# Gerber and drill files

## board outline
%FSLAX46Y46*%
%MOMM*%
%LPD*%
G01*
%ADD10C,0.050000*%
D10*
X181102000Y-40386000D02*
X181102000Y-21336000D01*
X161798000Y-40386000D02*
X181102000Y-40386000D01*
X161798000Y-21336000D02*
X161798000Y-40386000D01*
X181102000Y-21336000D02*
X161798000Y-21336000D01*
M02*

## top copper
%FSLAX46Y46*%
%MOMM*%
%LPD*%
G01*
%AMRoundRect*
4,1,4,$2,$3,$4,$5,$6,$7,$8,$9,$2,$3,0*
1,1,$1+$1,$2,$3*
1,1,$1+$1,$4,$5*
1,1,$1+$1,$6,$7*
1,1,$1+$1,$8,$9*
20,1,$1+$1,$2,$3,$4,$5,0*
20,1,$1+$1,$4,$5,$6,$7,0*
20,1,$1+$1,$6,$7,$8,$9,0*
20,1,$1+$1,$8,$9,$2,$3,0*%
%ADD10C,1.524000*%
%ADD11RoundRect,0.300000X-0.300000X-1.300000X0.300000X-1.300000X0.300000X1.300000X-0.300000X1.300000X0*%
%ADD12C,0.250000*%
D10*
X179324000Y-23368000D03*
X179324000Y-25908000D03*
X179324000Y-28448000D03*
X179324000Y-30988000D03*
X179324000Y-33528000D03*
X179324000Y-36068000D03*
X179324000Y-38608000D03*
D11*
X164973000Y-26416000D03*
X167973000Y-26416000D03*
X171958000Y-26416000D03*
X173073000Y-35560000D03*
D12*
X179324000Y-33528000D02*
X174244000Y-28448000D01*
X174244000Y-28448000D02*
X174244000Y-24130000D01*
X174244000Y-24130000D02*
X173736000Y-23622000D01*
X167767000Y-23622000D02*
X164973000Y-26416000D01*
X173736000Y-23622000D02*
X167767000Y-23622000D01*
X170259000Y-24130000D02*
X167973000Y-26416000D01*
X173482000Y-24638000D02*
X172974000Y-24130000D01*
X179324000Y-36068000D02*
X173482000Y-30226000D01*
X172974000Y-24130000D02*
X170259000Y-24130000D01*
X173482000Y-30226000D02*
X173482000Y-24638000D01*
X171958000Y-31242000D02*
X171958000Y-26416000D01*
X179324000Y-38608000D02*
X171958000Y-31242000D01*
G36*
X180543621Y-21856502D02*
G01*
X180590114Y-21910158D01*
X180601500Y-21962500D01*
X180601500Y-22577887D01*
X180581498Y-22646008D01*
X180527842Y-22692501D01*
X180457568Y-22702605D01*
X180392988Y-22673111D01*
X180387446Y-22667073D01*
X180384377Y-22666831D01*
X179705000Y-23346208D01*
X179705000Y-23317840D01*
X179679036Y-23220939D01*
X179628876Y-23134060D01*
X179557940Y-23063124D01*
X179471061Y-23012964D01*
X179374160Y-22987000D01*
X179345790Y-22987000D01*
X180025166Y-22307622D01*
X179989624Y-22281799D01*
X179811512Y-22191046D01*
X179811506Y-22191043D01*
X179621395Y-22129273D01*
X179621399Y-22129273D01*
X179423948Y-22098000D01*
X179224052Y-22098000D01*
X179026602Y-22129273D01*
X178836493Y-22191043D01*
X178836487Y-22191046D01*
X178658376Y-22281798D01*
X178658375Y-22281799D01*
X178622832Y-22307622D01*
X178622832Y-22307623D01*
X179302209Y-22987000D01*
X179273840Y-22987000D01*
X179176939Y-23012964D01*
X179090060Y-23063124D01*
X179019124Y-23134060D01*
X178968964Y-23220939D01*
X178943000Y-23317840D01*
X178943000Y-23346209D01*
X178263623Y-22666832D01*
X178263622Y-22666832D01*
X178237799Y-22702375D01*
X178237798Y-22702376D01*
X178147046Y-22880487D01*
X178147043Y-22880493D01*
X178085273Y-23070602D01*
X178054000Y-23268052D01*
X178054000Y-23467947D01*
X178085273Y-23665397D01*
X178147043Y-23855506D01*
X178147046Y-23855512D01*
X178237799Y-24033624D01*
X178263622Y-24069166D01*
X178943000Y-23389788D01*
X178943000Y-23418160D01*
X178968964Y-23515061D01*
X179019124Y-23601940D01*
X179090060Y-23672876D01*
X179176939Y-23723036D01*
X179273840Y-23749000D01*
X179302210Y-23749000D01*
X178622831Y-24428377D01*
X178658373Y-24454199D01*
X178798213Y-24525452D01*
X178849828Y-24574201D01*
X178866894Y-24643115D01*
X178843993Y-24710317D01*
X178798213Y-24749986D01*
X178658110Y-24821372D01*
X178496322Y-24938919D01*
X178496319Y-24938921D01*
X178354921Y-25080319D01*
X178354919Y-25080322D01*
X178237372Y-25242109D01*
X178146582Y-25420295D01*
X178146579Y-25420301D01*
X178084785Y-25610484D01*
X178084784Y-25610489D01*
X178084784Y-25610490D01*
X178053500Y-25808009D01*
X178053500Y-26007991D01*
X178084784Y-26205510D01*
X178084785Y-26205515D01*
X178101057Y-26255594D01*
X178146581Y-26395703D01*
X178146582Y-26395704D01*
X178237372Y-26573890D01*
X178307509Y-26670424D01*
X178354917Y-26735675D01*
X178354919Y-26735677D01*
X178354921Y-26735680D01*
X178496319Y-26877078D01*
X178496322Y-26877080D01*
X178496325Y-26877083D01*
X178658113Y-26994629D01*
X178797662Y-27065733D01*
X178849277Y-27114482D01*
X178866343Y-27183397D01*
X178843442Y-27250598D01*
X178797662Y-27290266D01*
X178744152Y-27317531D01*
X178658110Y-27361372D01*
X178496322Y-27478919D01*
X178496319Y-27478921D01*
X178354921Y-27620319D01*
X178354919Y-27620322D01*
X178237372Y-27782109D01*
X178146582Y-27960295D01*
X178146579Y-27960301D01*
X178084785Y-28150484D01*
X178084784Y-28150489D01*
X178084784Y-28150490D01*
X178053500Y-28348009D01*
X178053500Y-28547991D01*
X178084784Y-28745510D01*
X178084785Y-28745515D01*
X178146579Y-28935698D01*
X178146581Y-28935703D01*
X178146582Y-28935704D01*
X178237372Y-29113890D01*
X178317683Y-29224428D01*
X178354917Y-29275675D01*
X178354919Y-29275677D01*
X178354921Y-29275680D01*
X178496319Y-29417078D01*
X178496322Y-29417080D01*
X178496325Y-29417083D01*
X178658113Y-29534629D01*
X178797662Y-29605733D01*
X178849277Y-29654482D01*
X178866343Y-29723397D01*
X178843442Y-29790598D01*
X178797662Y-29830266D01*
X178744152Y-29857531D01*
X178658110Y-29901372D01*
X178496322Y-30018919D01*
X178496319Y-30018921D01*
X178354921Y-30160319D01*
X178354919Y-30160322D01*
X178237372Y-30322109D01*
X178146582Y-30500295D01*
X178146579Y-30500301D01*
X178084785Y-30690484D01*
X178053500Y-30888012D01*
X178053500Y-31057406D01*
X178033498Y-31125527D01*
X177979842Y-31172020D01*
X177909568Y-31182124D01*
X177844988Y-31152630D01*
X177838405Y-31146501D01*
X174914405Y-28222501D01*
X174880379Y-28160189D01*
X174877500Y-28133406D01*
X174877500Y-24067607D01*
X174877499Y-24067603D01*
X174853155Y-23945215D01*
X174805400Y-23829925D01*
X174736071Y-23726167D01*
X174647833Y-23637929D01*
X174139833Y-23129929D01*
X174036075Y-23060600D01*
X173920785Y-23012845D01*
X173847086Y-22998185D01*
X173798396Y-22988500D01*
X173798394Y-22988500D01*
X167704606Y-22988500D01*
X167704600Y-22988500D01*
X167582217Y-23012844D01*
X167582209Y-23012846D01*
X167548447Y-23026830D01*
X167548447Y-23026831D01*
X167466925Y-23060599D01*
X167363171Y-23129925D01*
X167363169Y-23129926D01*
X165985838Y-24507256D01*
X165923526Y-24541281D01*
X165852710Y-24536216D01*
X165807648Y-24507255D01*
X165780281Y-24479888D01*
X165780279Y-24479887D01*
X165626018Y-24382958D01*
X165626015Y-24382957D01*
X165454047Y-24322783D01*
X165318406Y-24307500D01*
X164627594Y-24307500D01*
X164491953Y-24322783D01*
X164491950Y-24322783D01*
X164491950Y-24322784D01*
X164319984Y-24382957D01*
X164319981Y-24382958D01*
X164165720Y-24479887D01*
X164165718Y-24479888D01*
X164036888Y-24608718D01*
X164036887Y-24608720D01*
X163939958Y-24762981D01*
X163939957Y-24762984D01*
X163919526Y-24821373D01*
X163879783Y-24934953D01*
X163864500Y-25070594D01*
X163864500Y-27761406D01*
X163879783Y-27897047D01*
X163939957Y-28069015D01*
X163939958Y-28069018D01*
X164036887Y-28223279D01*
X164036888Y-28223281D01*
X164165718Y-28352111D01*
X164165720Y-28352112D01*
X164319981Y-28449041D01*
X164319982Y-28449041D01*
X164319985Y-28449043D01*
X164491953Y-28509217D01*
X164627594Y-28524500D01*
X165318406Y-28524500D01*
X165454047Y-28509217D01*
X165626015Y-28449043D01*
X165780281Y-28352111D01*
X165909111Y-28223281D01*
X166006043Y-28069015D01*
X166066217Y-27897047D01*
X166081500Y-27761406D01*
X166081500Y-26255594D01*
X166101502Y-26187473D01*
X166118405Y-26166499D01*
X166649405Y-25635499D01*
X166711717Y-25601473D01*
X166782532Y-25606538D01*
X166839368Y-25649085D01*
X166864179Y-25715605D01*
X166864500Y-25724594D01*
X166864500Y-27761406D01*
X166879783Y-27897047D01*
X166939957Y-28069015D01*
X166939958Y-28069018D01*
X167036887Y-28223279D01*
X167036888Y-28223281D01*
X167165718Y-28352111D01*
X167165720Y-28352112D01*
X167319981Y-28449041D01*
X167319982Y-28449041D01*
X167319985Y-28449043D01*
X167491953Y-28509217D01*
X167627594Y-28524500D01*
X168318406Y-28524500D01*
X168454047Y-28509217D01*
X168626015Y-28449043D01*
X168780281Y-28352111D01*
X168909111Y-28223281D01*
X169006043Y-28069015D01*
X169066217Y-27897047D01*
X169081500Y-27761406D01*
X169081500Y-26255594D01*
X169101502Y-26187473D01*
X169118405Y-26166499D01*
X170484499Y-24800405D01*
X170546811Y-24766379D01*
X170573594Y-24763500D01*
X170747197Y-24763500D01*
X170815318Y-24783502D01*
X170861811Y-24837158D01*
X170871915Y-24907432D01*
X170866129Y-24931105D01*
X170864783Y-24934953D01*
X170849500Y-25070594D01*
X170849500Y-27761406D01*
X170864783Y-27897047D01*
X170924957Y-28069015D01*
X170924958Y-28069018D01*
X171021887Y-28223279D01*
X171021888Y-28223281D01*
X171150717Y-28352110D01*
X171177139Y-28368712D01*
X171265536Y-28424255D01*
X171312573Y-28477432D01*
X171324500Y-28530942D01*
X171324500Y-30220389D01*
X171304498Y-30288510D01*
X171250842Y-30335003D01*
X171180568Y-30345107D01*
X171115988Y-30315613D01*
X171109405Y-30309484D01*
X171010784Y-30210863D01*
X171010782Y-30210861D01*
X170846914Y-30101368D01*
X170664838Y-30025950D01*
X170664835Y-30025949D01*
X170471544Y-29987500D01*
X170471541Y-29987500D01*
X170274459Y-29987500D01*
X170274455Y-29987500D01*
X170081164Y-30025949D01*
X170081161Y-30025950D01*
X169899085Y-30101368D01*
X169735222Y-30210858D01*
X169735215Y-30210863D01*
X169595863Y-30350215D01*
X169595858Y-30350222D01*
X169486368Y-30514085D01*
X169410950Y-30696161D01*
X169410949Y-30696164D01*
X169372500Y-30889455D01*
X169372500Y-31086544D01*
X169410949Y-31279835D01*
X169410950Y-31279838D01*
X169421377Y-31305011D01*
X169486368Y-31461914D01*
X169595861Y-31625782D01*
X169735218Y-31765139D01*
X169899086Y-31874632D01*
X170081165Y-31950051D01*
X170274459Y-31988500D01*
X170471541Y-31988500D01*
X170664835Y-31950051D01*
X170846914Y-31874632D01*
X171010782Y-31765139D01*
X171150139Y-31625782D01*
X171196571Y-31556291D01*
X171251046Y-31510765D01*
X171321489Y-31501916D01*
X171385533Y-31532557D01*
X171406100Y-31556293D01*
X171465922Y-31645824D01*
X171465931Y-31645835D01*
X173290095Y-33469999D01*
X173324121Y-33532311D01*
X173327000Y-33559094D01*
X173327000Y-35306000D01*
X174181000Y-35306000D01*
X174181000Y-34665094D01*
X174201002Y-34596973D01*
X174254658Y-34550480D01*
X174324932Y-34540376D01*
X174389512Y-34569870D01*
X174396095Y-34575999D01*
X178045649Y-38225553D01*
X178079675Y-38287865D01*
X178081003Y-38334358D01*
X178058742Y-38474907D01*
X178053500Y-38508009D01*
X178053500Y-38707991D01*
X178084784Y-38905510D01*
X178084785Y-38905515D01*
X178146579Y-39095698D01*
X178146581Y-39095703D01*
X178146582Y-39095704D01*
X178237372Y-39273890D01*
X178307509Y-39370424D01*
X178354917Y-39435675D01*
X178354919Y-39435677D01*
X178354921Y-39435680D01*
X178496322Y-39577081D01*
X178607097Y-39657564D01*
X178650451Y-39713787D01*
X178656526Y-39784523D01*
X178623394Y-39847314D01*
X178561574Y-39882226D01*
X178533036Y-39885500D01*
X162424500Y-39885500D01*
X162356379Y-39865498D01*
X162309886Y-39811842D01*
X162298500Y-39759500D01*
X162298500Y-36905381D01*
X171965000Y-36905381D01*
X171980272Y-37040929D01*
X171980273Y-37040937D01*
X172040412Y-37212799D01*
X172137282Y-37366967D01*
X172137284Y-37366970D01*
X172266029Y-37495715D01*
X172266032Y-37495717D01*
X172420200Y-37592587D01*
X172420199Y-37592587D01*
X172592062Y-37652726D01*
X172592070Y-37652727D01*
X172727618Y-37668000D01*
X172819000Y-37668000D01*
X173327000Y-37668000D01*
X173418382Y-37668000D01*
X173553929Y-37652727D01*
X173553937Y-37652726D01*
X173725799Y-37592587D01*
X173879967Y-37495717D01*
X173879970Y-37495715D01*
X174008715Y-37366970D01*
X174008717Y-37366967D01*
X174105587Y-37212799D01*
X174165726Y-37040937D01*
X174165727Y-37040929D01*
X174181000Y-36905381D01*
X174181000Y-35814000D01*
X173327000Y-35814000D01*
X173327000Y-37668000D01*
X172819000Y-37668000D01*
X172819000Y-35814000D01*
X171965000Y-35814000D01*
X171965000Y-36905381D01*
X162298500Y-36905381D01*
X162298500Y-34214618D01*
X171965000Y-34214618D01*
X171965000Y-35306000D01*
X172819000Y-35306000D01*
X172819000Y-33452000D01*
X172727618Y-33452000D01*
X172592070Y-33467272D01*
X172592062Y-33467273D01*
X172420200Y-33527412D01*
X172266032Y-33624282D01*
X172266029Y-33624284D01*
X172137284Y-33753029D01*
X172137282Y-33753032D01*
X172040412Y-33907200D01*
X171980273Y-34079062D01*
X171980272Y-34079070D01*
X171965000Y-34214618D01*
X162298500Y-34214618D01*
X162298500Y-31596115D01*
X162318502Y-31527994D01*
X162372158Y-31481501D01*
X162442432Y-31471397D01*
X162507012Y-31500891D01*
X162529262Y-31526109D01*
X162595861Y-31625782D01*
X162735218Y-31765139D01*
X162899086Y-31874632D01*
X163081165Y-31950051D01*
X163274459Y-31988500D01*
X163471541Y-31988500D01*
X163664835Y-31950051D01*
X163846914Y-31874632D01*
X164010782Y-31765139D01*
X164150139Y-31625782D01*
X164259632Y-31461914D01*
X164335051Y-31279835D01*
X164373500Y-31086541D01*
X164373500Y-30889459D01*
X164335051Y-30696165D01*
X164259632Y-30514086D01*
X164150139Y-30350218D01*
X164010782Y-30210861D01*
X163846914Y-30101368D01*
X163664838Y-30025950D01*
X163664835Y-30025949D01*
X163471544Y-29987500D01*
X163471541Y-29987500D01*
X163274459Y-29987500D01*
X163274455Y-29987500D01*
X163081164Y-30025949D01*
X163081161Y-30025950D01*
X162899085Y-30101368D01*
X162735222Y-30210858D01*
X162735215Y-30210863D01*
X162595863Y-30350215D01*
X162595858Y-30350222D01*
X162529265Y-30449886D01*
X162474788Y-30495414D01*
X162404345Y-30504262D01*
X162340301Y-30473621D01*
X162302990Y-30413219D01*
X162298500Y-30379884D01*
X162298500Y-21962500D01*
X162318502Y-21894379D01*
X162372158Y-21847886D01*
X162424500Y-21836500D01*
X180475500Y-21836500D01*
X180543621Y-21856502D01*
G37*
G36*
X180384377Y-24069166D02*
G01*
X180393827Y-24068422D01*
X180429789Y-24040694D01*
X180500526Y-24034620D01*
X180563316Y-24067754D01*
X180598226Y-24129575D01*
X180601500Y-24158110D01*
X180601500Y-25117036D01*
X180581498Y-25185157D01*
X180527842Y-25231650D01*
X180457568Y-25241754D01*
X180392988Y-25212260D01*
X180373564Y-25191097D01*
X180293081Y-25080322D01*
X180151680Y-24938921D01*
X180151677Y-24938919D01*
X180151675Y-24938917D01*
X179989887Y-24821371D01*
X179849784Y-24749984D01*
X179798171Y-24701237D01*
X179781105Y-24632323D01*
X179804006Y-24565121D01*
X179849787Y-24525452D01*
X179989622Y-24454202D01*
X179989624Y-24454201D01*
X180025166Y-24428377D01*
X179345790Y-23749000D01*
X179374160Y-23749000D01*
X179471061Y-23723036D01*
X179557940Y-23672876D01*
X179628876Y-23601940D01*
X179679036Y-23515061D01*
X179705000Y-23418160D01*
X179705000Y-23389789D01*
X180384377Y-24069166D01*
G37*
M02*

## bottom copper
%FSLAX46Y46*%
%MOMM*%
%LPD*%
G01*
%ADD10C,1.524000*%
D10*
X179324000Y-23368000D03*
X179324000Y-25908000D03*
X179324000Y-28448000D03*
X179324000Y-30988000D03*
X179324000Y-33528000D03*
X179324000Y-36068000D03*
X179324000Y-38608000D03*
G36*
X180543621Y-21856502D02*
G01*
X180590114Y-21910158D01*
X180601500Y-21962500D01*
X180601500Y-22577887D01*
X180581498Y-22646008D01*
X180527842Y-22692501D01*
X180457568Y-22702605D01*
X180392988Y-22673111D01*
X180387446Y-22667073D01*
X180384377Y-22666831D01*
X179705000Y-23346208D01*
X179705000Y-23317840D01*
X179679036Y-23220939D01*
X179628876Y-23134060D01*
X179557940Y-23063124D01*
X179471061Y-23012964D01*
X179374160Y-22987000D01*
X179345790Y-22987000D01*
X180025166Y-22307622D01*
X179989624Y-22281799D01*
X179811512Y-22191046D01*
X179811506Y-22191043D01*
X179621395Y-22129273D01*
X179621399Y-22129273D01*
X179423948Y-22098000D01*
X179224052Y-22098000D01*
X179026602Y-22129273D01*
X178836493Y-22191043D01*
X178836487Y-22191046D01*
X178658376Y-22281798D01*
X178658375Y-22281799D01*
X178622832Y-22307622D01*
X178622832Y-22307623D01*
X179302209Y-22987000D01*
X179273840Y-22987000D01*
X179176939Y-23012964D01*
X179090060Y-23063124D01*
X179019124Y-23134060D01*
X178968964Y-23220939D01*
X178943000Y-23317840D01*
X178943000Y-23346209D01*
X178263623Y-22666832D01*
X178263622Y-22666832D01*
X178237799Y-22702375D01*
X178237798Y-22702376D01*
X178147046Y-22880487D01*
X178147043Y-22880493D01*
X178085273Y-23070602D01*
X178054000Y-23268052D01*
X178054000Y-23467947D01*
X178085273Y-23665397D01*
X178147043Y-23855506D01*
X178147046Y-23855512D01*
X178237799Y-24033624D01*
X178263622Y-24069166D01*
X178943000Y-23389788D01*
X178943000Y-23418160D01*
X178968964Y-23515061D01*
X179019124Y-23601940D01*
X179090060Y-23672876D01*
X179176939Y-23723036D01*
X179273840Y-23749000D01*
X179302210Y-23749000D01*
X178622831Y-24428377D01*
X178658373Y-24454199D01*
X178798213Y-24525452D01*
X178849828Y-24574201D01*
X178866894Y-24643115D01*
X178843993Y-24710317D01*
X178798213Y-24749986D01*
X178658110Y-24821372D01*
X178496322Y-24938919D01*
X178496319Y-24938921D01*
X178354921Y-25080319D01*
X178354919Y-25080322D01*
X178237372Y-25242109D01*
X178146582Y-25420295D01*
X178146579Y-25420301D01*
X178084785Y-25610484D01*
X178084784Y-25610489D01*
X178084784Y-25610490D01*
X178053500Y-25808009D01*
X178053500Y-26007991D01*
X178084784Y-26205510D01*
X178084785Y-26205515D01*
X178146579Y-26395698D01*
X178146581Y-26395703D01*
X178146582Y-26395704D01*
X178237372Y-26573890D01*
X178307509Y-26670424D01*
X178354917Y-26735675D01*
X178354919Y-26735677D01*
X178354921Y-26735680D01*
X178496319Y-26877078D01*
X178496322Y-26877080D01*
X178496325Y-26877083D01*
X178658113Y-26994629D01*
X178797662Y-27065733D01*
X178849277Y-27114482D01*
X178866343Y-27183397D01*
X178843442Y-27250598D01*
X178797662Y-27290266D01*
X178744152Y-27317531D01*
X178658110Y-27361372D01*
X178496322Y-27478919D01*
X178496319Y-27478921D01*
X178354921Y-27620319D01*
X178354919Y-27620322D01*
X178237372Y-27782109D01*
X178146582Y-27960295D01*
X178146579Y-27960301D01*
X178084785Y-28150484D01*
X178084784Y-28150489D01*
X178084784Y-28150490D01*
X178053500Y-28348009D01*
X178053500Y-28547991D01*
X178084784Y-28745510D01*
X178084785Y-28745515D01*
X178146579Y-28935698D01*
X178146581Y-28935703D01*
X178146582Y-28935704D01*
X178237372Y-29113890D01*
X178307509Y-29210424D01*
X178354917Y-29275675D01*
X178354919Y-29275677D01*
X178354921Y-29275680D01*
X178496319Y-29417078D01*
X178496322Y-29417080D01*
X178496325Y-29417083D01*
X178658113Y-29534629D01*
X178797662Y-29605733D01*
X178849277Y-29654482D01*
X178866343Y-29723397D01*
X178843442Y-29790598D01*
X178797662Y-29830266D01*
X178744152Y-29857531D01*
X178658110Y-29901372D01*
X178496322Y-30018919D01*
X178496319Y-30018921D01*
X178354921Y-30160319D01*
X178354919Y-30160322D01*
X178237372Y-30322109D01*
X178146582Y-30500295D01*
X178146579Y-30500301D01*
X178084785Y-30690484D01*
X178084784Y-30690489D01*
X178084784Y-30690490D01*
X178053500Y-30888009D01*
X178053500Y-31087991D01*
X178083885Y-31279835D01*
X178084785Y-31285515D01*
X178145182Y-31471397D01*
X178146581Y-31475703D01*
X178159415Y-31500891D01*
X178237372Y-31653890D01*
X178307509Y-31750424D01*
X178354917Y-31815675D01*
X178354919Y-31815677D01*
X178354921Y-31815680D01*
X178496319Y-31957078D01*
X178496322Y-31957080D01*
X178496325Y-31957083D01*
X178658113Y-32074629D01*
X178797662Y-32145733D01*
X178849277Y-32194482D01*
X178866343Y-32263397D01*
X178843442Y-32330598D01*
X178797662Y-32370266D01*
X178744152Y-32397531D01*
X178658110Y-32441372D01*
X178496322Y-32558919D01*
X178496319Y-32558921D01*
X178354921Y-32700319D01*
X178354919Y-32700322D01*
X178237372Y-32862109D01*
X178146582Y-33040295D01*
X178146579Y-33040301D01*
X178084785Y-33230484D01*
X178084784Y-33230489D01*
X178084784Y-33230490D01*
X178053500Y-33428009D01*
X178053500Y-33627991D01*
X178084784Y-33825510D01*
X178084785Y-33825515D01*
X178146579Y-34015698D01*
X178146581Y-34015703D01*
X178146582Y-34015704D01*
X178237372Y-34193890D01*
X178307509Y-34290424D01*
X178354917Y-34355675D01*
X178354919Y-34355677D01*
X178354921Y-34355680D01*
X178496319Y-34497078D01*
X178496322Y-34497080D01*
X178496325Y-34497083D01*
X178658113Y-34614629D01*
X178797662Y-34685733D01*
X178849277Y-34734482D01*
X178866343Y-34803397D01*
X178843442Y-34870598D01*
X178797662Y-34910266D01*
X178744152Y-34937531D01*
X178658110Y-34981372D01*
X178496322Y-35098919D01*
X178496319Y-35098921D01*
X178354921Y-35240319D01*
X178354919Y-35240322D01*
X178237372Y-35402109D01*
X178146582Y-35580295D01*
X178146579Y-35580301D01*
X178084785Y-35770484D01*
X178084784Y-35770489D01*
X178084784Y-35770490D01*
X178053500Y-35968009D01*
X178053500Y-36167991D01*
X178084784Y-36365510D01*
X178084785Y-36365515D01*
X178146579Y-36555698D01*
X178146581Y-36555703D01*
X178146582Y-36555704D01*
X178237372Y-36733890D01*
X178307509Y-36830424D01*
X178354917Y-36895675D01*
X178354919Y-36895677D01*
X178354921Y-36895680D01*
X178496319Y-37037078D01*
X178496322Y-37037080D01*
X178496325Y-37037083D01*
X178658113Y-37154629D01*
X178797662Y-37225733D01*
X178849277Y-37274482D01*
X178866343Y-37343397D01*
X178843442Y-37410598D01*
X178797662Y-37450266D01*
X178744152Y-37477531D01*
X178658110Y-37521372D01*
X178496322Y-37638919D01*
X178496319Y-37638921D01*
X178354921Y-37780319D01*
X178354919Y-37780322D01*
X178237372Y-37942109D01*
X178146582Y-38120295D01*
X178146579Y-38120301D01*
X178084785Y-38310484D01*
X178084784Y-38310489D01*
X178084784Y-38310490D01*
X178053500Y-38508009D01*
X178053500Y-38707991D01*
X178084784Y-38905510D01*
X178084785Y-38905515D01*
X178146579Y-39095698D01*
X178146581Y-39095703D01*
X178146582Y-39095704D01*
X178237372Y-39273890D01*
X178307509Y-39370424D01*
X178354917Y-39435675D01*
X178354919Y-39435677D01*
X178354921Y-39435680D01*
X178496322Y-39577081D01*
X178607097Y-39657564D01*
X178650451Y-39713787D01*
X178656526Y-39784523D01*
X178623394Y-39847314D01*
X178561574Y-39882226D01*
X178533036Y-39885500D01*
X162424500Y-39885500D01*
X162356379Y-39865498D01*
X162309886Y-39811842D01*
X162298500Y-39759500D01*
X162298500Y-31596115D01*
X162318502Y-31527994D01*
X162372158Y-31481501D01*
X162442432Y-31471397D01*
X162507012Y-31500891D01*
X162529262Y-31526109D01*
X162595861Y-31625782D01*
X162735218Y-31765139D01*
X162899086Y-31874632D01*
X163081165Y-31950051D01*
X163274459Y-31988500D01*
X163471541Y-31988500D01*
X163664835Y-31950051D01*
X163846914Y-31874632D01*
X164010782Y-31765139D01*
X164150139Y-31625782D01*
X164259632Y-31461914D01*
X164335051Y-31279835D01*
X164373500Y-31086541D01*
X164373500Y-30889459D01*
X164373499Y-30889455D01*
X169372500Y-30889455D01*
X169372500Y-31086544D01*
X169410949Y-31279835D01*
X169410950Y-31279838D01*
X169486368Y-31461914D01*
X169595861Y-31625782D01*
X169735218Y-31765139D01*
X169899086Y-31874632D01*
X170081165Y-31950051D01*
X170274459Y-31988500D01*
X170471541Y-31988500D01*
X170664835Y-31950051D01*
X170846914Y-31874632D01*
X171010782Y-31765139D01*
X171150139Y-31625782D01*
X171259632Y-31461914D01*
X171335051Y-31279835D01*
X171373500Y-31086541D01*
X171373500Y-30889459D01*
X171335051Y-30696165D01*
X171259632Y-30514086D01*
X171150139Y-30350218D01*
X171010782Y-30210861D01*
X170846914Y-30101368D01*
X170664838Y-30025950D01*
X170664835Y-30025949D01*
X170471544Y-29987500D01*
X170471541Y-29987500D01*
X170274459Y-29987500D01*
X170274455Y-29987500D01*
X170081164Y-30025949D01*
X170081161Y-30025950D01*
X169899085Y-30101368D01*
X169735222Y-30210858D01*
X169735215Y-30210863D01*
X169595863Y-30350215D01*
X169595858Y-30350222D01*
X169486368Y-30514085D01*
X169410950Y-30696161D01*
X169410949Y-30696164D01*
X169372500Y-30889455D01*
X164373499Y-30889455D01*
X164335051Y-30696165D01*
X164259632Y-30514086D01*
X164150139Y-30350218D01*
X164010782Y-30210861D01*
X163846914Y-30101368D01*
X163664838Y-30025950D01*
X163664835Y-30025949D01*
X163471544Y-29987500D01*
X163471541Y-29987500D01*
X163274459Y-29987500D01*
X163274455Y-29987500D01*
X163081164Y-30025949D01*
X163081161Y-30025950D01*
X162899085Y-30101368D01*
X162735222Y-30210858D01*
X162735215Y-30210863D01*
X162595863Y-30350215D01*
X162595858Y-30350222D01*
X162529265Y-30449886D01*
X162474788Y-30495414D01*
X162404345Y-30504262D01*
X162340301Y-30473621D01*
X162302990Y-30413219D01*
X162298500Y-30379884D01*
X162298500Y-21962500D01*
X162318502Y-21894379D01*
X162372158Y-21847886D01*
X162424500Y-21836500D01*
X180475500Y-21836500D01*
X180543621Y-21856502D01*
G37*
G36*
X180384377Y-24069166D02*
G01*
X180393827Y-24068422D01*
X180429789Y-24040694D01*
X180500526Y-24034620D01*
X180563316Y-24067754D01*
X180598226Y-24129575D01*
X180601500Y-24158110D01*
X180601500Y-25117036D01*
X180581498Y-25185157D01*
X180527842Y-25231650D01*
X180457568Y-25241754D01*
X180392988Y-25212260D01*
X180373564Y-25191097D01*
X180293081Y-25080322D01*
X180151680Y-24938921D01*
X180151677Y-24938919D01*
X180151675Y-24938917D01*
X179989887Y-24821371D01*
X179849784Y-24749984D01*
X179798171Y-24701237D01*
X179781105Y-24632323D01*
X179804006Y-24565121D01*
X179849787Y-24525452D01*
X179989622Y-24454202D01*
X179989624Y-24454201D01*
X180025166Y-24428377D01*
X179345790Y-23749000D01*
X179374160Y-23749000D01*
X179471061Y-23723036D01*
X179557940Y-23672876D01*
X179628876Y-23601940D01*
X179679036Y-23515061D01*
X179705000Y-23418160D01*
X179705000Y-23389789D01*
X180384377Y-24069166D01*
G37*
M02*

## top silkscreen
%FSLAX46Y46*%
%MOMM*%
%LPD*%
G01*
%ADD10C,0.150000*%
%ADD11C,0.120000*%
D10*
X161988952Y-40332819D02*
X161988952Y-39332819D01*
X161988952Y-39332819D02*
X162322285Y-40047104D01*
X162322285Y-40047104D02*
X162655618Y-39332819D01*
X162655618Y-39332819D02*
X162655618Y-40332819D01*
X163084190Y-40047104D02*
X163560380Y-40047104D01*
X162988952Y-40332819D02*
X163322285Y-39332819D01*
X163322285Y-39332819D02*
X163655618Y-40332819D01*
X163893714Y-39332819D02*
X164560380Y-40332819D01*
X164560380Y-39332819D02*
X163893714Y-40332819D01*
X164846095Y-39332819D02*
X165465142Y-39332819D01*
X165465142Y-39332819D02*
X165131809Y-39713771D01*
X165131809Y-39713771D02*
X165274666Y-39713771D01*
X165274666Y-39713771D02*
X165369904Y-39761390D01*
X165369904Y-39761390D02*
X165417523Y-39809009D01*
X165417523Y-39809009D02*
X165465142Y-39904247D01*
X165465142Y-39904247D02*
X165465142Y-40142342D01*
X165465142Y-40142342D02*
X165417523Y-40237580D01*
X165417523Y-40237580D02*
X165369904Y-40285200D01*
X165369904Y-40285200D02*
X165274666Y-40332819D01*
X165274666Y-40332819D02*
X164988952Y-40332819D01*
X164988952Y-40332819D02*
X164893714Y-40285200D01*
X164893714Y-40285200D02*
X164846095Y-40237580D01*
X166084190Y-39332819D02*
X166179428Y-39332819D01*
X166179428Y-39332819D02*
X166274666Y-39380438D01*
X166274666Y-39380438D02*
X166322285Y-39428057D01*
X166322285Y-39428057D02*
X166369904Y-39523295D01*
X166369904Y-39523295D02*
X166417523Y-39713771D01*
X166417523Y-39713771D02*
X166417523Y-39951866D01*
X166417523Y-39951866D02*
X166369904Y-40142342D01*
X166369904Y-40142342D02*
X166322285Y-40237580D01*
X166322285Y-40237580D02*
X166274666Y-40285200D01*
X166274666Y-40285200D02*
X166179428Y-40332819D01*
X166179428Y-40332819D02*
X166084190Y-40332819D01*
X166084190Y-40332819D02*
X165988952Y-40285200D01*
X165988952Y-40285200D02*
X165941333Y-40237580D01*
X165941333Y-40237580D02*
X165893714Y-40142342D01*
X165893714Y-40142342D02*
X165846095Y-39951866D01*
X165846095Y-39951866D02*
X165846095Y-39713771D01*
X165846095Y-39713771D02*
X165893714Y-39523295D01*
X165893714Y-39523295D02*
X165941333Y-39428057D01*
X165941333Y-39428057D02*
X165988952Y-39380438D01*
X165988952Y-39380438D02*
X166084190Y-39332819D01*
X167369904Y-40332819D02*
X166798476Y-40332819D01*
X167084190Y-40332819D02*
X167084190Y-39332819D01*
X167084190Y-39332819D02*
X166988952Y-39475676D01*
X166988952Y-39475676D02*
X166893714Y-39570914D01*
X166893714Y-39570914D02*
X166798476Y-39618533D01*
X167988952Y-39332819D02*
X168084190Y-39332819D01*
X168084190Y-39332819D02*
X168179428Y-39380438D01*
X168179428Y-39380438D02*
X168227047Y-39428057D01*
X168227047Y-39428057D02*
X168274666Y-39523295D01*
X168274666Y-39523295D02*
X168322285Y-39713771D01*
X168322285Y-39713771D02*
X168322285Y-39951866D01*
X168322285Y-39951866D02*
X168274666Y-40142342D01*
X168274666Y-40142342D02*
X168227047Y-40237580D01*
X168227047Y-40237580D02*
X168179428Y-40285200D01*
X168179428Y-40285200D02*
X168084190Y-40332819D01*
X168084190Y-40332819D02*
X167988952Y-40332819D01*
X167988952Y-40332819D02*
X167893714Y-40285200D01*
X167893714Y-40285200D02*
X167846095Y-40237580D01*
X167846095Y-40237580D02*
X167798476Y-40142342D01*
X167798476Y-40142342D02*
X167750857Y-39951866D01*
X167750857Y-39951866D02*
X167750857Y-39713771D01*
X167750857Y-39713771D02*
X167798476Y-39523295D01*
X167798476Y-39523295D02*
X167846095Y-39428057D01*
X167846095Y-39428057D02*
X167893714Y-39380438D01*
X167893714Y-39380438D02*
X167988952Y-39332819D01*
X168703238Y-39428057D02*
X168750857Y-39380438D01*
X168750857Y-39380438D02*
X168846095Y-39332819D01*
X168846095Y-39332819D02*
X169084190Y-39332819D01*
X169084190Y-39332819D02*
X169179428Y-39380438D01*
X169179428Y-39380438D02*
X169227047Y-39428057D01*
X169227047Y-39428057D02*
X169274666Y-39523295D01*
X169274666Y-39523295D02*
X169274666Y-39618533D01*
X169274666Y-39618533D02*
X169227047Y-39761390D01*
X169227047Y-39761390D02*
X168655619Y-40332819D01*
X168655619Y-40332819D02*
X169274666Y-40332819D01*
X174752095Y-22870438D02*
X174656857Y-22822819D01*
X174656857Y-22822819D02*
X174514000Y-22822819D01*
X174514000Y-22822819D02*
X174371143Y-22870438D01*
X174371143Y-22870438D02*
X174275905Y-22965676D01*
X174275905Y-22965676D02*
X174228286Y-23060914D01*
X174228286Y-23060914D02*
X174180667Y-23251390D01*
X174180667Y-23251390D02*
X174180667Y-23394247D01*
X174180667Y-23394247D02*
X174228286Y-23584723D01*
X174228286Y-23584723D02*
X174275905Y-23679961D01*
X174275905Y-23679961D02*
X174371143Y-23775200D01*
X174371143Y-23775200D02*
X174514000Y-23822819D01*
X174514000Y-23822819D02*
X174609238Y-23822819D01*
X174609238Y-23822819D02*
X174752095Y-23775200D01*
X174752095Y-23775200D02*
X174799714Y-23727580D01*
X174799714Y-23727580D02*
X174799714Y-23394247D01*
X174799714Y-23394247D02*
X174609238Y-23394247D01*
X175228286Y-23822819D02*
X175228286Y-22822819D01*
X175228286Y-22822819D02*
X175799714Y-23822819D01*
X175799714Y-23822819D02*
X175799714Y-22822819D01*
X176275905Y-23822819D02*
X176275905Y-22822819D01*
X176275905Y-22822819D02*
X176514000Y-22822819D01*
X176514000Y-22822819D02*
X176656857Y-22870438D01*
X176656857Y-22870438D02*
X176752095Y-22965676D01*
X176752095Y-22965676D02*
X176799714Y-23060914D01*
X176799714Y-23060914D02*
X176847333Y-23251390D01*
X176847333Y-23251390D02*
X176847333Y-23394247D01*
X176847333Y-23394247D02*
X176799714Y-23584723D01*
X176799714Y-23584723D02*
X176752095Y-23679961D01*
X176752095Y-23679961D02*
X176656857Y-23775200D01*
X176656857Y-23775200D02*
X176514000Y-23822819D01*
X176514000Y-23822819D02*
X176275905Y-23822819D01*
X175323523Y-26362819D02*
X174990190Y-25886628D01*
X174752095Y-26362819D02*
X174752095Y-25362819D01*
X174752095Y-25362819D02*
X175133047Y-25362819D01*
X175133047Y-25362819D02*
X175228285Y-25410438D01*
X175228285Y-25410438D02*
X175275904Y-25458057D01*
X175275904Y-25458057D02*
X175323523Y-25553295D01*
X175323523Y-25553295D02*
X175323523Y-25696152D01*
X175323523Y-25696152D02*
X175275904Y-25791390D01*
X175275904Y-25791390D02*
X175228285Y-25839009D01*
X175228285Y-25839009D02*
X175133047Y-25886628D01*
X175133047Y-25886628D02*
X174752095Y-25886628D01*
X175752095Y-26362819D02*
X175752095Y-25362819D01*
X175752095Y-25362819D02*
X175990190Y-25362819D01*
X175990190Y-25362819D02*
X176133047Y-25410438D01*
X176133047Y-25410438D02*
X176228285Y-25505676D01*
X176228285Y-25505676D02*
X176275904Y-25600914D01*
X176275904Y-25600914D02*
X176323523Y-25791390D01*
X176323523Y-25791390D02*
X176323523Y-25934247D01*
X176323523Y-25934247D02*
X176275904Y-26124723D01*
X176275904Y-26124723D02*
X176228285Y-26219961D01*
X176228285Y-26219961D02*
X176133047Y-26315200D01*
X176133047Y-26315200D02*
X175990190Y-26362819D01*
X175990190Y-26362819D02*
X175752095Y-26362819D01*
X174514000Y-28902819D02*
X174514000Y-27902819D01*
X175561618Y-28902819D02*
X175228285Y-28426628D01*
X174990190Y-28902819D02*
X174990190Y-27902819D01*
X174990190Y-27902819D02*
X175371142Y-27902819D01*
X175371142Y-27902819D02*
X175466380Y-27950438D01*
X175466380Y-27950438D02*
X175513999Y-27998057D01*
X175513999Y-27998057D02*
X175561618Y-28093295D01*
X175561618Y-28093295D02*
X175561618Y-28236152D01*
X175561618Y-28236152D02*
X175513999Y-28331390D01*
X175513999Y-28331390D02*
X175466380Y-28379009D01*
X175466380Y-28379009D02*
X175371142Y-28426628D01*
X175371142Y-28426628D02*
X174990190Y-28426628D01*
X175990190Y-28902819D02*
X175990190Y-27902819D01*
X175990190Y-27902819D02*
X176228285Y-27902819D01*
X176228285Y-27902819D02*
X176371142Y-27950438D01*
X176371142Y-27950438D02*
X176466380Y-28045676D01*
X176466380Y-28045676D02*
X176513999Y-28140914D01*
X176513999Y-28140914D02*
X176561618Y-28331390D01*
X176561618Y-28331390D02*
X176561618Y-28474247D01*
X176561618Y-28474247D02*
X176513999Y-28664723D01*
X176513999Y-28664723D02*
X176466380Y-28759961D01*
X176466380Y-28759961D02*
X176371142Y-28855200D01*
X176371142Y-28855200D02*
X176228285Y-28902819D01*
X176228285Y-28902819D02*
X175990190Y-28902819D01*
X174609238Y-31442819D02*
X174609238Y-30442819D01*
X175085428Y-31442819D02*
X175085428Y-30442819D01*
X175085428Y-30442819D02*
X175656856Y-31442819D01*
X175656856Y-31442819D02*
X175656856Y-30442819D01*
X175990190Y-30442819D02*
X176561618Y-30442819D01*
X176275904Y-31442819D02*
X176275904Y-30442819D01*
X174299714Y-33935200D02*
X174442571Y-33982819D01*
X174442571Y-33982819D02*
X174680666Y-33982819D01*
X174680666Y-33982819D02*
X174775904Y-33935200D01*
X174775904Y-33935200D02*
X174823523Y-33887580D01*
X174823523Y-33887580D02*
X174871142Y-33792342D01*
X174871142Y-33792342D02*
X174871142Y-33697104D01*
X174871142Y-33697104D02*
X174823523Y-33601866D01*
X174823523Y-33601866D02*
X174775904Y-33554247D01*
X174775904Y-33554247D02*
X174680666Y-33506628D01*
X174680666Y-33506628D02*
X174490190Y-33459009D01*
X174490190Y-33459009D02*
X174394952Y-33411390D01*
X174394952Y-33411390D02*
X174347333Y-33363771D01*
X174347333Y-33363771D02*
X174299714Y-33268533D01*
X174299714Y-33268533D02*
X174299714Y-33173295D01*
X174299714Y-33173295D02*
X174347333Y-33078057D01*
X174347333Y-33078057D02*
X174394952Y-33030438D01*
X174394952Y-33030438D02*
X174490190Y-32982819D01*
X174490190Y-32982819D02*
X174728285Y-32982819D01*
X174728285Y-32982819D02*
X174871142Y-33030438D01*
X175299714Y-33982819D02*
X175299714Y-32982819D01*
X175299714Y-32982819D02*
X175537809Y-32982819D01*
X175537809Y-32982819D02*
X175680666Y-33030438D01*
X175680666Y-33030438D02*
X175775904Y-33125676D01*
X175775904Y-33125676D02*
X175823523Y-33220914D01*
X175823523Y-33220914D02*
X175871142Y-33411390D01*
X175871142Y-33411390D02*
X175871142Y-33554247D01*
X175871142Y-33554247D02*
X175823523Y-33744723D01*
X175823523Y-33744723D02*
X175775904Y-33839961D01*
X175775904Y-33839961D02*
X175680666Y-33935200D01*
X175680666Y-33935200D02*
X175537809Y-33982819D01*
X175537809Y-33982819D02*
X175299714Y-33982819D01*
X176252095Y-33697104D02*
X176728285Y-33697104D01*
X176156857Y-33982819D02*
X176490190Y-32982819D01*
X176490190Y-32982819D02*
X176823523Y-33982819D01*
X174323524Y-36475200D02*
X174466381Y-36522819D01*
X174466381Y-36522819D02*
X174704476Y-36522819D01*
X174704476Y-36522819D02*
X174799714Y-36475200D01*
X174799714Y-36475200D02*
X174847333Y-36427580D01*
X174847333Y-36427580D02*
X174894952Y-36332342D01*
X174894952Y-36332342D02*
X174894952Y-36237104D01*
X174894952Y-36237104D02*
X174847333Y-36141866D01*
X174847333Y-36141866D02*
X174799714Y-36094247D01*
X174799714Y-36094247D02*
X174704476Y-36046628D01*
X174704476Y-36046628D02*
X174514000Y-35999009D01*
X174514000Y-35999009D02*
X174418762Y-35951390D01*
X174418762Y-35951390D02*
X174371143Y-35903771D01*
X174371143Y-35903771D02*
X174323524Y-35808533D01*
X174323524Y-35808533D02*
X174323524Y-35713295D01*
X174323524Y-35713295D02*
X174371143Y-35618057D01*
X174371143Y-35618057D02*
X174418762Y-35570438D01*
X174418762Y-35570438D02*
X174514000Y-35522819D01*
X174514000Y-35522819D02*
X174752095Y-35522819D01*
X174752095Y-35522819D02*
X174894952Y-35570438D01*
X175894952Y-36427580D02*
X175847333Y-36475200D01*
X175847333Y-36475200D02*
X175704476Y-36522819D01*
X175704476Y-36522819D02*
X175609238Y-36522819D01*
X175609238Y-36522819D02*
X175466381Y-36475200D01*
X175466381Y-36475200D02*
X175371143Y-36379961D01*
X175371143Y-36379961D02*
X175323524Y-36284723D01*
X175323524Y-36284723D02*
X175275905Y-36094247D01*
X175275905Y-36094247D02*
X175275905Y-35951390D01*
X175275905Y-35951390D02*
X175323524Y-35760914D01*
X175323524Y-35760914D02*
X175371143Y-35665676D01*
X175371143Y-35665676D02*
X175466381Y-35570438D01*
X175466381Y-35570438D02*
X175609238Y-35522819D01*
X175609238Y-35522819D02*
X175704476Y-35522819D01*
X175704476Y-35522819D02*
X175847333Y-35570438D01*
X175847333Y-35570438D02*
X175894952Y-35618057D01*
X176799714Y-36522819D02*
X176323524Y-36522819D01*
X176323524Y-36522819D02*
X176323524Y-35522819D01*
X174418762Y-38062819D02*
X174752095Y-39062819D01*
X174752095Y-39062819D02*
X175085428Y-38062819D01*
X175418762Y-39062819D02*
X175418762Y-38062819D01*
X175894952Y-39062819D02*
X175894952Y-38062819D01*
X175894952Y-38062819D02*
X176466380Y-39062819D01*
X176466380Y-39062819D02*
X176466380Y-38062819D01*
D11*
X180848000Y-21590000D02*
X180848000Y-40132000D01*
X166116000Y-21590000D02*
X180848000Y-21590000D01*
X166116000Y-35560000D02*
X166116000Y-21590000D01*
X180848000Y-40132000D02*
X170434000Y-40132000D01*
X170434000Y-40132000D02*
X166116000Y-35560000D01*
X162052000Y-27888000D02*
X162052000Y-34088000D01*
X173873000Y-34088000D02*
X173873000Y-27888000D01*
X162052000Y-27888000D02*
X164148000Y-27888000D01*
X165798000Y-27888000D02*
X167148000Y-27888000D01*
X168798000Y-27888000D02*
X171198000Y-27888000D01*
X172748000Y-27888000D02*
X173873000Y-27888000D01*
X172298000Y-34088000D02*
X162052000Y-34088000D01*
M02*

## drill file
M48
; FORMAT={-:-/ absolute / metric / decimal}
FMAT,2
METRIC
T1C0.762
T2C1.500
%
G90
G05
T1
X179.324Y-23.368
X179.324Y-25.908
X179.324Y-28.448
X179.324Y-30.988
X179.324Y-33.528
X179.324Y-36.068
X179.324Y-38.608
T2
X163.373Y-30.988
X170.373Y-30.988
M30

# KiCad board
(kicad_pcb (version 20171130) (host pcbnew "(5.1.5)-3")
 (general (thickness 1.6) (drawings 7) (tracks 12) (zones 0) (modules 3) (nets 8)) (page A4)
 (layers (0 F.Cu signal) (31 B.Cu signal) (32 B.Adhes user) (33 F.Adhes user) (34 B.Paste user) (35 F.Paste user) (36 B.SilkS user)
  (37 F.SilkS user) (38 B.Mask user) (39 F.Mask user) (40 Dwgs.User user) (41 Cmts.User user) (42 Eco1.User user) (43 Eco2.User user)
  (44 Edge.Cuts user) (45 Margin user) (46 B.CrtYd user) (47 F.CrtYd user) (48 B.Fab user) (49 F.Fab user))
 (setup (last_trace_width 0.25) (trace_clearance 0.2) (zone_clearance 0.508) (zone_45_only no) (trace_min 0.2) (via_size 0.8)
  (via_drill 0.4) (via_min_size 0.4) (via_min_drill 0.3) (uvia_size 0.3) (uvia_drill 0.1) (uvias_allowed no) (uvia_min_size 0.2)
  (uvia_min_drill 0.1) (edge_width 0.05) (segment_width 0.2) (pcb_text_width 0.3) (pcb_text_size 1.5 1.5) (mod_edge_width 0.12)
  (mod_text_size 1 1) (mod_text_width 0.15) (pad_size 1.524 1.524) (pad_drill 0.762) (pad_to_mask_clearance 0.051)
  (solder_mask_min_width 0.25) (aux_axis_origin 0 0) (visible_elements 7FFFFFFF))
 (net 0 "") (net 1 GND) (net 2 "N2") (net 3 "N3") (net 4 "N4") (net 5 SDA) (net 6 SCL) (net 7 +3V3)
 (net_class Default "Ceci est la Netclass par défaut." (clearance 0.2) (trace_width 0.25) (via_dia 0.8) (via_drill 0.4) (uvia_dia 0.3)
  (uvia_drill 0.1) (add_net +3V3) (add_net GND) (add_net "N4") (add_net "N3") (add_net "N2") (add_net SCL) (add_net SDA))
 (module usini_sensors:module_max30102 (layer F.Cu) (at 181.864 20.828 180)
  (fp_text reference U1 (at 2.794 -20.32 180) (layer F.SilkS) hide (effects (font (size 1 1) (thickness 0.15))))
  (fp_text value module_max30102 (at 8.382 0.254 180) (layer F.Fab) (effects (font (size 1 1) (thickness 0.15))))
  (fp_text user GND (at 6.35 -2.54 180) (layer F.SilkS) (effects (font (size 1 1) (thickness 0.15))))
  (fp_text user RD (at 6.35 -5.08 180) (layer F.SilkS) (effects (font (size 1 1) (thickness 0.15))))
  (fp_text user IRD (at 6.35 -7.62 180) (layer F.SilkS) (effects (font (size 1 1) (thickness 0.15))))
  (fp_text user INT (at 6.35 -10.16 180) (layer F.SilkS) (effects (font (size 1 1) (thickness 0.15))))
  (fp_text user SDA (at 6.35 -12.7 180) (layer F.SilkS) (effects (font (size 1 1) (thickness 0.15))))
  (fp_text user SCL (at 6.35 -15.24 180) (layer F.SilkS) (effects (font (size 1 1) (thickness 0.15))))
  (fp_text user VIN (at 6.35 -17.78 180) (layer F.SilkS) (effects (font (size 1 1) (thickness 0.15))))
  (fp_line (start 1.016 -0.762) (end 1.016 -19.304) (layer F.SilkS) (width 0.12))
  (fp_line (start 15.748 -0.762) (end 1.016 -0.762) (layer F.SilkS) (width 0.12))
  (fp_line (start 15.748 -14.732) (end 15.748 -0.762) (layer F.SilkS) (width 0.12))
  (fp_line (start 1.016 -19.304) (end 11.43 -19.304) (layer F.SilkS) (width 0.12))
  (fp_line (start 11.43 -19.304) (end 15.748 -14.732) (layer F.SilkS) (width 0.12))
  (pad 7 thru_hole circle (at 2.54 -2.54 180) (size 1.524 1.524) (drill 0.762) (layers *.Cu *.Mask) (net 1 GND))
  (pad 6 thru_hole circle (at 2.54 -5.08 180) (size 1.524 1.524) (drill 0.762) (layers *.Cu *.Mask) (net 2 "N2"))
  (pad 5 thru_hole circle (at 2.54 -7.62 180) (size 1.524 1.524) (drill 0.762) (layers *.Cu *.Mask) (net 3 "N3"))
  (pad 4 thru_hole circle (at 2.54 -10.16 180) (size 1.524 1.524) (drill 0.762) (layers *.Cu *.Mask) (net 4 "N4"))
  (pad 3 thru_hole circle (at 2.54 -12.7 180) (size 1.524 1.524) (drill 0.762) (layers *.Cu *.Mask) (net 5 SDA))
  (pad 2 thru_hole circle (at 2.54 -15.24 180) (size 1.524 1.524) (drill 0.762) (layers *.Cu *.Mask) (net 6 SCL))
  (pad 1 thru_hole circle (at 2.54 -17.78 180) (size 1.524 1.524) (drill 0.762) (layers *.Cu *.Mask) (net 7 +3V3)))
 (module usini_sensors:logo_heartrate (layer B.Cu) (at 173.99 24.13 180)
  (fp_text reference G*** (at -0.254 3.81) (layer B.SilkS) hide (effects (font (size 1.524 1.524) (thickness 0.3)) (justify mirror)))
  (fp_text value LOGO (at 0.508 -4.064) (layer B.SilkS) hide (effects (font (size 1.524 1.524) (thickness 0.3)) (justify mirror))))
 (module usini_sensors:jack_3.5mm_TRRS (layer F.Cu) (at 168.148 30.988)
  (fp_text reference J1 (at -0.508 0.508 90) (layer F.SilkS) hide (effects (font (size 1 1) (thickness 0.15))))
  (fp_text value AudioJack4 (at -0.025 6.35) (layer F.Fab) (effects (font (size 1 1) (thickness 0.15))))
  (fp_line (start -6.096 -3.1) (end -6.096 3.1) (layer F.SilkS) (width 0.12))
  (fp_line (start 5.725 3.1) (end 5.725 -3.1) (layer F.SilkS) (width 0.12))
  (fp_line (start -6.096 -3.1) (end -4 -3.1) (layer F.SilkS) (width 0.12))
  (fp_line (start -2.35 -3.1) (end -1 -3.1) (layer F.SilkS) (width 0.12))
  (fp_line (start 0.65 -3.1) (end 3.05 -3.1) (layer F.SilkS) (width 0.12))
  (fp_line (start 4.6 -3.1) (end 5.725 -3.1) (layer F.SilkS) (width 0.12))
  (fp_line (start 4.15 3.1) (end -6.096 3.1) (layer F.SilkS) (width 0.12))
  (pad "" np_thru_hole circle (at 2.225 0) (size 1.5 1.5) (drill 1.5) (layers *.Cu *.Mask))
  (pad "" np_thru_hole circle (at -4.775 0) (size 1.5 1.5) (drill 1.5) (layers *.Cu *.Mask))
  (pad R2 smd roundrect (at -3.175 -4.572) (size 1.2 3.2) (layers F.Cu F.Paste F.Mask) (roundrect_rratio 0.25) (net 5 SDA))
  (pad R1 smd roundrect (at -0.175 -4.572) (size 1.2 3.2) (layers F.Cu F.Paste F.Mask) (roundrect_rratio 0.25) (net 6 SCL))
  (pad T smd roundrect (at 3.81 -4.572) (size 1.2 3.2) (layers F.Cu F.Paste F.Mask) (roundrect_rratio 0.25) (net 7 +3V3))
  (pad S smd roundrect (at 4.925 4.572) (size 1.2 3.2) (layers F.Cu F.Paste F.Mask) (roundrect_rratio 0.25) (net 1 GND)))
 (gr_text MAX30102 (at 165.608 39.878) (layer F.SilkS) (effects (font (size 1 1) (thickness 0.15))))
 (gr_line (start 181.102 40.386) (end 181.102 21.336) (layer Edge.Cuts) (width 0.05))
 (gr_line (start 161.798 40.386) (end 181.102 40.386) (layer Edge.Cuts) (width 0.05))
 (gr_line (start 161.798 21.336) (end 161.798 40.386) (layer Edge.Cuts) (width 0.05))
 (gr_line (start 181.102 21.336) (end 161.798 21.336) (layer Edge.Cuts) (width 0.05))
 (segment (start 179.324 33.528) (end 174.244 28.448) (width 0.25) (layer F.Cu) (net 5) (status 10))
 (segment (start 174.244 28.448) (end 174.244 24.13) (width 0.25) (layer F.Cu) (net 5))
 (segment (start 174.244 24.13) (end 173.736 23.622) (width 0.25) (layer F.Cu) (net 5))
 (segment (start 167.767 23.622) (end 164.973 26.416) (width 0.25) (layer F.Cu) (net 5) (status 20))
 (segment (start 173.736 23.622) (end 167.767 23.622) (width 0.25) (layer F.Cu) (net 5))
 (segment (start 170.259 24.13) (end 167.973 26.416) (width 0.25) (layer F.Cu) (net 6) (status 20))
 (segment (start 173.482 24.638) (end 172.974 24.13) (width 0.25) (layer F.Cu) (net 6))
 (segment (start 179.324 36.068) (end 173.482 30.226) (width 0.25) (layer F.Cu) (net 6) (status 10))
 (segment (start 172.974 24.13) (end 170.259 24.13) (width 0.25) (layer F.Cu) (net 6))
 (segment (start 173.482 30.226) (end 173.482 24.638) (width 0.25) (layer F.Cu) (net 6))
 (segment (start 171.958 31.242) (end 171.958 26.416) (width 0.25) (layer F.Cu) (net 7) (status 20))
 (segment (start 179.324 38.608) (end 171.958 31.242) (width 0.25) (layer F.Cu) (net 7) (status 10))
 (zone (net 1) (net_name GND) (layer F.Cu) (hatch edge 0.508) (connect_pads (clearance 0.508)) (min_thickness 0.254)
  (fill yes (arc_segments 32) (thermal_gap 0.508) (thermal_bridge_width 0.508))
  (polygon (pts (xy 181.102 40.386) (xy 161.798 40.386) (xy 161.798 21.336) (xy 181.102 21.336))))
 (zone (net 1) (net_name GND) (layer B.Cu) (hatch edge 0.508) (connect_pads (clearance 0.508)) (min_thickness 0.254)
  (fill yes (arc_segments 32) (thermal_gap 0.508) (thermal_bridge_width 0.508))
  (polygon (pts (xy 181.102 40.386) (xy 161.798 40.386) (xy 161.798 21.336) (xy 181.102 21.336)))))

